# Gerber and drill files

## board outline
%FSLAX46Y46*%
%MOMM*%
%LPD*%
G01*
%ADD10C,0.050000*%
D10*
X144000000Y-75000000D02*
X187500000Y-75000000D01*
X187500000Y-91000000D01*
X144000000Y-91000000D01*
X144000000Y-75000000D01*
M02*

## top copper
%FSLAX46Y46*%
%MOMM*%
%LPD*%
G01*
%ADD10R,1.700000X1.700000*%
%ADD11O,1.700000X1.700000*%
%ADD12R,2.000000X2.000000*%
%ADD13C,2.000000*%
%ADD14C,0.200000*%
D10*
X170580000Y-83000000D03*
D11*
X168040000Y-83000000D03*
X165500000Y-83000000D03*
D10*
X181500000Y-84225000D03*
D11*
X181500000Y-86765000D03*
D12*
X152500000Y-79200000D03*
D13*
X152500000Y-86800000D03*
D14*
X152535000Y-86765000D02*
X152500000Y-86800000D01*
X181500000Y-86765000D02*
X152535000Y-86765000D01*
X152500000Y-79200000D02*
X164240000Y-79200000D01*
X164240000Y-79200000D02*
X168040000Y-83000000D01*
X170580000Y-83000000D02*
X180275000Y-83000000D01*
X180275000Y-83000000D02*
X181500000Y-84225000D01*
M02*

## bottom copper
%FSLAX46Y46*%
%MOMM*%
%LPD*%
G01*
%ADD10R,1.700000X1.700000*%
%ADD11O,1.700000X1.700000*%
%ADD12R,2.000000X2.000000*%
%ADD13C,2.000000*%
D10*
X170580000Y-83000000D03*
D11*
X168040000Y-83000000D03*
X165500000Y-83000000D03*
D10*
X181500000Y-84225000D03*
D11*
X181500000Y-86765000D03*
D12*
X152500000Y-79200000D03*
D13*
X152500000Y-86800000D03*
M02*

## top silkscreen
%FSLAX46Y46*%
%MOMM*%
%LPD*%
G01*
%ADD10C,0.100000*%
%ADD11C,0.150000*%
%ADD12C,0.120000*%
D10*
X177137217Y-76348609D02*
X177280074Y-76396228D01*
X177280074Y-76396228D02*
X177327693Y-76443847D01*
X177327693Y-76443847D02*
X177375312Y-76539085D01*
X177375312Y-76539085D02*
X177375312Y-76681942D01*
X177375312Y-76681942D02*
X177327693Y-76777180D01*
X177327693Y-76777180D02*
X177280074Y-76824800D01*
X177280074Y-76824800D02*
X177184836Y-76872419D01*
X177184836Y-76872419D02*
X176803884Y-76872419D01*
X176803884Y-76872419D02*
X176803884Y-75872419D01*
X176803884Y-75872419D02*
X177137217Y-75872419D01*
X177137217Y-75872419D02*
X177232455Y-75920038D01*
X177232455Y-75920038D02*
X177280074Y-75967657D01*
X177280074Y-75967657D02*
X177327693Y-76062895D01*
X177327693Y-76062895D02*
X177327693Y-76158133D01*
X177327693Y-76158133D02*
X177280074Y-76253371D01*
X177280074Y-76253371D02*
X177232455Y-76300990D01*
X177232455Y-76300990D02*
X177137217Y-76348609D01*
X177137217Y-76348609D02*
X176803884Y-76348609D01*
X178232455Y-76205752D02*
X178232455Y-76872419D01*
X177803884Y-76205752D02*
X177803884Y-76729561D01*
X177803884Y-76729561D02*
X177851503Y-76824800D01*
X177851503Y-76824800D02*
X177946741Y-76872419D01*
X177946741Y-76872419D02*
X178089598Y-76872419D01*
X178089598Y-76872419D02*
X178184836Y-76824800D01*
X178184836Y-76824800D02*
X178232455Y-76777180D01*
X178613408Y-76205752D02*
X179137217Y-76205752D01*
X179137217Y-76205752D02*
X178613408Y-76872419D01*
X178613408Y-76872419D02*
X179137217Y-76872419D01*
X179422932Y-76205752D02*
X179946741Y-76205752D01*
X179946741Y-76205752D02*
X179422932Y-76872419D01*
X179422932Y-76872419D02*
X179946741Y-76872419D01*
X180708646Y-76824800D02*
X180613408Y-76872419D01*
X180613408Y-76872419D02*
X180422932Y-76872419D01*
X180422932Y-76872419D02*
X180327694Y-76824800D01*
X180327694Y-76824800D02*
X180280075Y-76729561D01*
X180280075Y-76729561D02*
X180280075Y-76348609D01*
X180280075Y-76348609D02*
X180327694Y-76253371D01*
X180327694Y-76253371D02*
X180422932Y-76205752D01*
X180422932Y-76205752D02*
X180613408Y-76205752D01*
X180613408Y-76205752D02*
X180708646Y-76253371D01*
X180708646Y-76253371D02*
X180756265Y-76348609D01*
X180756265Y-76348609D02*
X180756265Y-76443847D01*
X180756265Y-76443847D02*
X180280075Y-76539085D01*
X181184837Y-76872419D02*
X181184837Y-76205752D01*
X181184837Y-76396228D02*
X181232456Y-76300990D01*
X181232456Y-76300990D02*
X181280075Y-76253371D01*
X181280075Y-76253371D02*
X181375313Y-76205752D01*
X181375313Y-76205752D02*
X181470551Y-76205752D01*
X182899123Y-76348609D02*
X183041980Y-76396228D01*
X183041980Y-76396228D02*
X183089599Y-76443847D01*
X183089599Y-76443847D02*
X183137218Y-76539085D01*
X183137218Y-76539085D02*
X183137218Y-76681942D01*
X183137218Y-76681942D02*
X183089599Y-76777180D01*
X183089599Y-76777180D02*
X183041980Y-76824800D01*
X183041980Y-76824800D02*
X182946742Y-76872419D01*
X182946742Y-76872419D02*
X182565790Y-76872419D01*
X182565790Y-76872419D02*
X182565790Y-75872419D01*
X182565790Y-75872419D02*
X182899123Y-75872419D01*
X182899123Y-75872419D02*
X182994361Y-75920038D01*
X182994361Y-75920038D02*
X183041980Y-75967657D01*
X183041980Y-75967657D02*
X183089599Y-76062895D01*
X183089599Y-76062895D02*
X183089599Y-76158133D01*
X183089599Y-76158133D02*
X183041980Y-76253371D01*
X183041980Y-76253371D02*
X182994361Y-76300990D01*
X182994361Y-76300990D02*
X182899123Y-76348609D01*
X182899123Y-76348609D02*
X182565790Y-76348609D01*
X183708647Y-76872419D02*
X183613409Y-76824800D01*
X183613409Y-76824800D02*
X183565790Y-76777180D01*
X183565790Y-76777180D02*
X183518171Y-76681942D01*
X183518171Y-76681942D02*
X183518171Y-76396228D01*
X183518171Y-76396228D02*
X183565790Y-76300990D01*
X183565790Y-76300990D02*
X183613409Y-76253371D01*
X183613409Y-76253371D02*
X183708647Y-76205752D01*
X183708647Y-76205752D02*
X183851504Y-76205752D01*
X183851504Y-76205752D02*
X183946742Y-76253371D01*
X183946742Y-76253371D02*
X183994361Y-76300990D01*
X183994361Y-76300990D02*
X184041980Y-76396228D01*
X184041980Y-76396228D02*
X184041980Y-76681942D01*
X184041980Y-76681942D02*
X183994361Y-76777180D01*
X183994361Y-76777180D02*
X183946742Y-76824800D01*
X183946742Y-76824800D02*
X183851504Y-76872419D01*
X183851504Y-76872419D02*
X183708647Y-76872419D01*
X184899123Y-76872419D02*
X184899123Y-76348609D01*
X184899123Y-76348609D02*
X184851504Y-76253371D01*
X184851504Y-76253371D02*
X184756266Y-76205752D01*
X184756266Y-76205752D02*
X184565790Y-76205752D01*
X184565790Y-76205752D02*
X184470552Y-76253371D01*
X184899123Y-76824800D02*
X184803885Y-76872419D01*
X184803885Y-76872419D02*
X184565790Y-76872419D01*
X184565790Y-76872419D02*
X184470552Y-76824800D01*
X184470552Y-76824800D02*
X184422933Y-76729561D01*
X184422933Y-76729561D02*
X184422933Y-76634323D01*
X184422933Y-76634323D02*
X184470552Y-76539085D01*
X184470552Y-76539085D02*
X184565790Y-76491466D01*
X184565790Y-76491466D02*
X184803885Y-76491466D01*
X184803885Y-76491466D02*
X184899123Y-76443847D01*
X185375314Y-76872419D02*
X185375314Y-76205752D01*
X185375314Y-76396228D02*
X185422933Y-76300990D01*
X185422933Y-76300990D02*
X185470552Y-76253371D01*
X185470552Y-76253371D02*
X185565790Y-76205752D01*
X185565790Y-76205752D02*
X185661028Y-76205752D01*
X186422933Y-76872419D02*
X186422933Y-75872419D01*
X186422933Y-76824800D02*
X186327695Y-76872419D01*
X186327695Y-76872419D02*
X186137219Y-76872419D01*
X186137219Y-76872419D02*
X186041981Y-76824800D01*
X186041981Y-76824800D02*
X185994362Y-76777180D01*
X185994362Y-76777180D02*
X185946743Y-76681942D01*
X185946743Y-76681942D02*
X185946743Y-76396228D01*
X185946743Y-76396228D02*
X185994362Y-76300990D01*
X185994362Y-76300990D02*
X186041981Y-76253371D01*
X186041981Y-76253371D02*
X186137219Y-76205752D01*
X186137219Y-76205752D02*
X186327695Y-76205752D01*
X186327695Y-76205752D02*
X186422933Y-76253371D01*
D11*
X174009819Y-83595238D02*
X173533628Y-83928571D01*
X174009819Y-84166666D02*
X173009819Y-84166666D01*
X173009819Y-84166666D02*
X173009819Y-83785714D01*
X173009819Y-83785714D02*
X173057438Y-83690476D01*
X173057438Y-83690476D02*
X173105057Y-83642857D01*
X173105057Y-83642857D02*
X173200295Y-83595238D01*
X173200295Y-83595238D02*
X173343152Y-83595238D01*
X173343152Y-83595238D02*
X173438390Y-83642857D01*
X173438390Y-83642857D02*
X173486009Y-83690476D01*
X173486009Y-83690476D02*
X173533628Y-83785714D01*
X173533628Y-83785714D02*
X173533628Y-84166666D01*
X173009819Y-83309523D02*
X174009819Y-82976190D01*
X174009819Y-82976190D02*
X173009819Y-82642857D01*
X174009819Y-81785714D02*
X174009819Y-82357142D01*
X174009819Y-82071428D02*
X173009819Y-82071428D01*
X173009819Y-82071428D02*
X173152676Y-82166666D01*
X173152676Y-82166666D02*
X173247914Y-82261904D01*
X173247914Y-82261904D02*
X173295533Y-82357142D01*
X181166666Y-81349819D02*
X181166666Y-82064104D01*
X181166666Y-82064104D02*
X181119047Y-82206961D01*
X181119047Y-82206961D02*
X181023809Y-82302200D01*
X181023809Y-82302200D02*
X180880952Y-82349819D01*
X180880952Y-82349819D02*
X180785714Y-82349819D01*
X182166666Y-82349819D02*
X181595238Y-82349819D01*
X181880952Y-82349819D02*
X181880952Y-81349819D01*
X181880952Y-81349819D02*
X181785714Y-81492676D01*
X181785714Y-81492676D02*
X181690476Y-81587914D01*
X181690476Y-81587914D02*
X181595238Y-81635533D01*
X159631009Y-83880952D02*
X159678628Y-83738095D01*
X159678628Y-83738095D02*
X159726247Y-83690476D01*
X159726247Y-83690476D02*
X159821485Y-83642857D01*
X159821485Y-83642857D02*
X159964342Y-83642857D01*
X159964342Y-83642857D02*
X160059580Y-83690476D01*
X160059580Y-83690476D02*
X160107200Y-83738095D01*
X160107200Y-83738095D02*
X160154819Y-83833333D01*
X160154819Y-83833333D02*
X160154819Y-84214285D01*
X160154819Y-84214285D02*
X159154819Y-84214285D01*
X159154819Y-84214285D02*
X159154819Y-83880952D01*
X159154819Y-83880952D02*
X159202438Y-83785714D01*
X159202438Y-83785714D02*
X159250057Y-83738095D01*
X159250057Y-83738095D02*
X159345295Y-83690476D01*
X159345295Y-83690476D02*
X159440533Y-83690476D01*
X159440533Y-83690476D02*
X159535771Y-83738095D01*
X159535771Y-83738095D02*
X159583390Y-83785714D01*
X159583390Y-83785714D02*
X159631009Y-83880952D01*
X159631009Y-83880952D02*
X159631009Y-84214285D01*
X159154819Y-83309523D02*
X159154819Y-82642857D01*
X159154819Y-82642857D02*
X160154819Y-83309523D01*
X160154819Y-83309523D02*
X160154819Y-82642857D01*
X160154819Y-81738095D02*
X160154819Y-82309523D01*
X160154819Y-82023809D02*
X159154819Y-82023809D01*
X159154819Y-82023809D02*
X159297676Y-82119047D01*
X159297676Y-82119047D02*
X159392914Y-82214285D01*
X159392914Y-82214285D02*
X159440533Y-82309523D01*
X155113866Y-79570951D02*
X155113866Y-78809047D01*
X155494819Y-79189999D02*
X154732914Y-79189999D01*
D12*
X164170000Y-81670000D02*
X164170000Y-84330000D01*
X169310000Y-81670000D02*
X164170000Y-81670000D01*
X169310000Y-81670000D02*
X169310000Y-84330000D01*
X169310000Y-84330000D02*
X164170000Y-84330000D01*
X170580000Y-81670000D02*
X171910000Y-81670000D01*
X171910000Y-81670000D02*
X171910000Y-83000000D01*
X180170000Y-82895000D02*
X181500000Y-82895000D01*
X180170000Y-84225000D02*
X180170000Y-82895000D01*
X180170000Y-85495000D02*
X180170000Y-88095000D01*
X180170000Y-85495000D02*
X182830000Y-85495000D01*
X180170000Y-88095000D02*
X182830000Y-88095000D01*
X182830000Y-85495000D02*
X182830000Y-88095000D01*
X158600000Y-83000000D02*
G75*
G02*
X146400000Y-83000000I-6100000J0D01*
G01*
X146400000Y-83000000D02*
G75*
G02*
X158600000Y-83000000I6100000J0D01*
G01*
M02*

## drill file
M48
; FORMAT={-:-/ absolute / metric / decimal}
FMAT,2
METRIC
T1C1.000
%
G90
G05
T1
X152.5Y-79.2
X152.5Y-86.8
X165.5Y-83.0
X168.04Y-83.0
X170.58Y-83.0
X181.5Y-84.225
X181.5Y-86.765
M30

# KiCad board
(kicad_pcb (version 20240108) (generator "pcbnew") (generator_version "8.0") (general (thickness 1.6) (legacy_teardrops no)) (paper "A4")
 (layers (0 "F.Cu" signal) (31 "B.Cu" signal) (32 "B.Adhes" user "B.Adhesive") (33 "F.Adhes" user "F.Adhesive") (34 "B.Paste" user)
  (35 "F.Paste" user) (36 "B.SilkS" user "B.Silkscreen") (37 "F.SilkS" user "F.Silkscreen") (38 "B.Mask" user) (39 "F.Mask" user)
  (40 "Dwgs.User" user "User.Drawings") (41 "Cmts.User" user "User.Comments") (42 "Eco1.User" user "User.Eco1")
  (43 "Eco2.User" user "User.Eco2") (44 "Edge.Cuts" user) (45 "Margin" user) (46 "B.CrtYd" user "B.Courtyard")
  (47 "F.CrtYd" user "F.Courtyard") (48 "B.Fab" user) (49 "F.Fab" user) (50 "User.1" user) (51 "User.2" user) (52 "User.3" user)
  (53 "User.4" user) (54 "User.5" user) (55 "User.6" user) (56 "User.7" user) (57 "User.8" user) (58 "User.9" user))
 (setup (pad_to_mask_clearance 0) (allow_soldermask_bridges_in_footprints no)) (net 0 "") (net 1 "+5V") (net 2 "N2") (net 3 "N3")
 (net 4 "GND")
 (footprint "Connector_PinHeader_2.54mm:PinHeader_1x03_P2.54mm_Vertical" (layer "F.Cu") (at 170.58 83 -90)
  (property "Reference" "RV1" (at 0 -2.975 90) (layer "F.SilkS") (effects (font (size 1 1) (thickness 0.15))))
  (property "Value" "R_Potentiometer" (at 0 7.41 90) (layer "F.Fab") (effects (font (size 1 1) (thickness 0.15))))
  (fp_line (start -1.33 6.41) (end 1.33 6.41) (stroke (width 0.12) (type solid)) (layer "F.SilkS"))
  (fp_line (start -1.33 1.27) (end -1.33 6.41) (stroke (width 0.12) (type solid)) (layer "F.SilkS"))
  (fp_line (start -1.33 1.27) (end 1.33 1.27) (stroke (width 0.12) (type solid)) (layer "F.SilkS"))
  (fp_line (start 1.33 1.27) (end 1.33 6.41) (stroke (width 0.12) (type solid)) (layer "F.SilkS"))
  (fp_line (start -1.33 0) (end -1.33 -1.33) (stroke (width 0.12) (type solid)) (layer "F.SilkS"))
  (fp_line (start -1.33 -1.33) (end 0 -1.33) (stroke (width 0.12) (type solid)) (layer "F.SilkS"))
  (pad "1" thru_hole rect (at 0 0 270) (size 1.7 1.7) (drill 1) (layers "*.Cu" "*.Mask") (remove_unused_layers no) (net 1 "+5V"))
  (pad "2" thru_hole oval (at 0 2.54 270) (size 1.7 1.7) (drill 1) (layers "*.Cu" "*.Mask") (remove_unused_layers no) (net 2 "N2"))
  (pad "3" thru_hole oval (at 0 5.08 270) (size 1.7 1.7) (drill 1) (layers "*.Cu" "*.Mask") (remove_unused_layers no) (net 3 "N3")))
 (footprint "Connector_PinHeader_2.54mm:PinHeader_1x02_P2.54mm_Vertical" (layer "F.Cu") (at 181.5 84.225)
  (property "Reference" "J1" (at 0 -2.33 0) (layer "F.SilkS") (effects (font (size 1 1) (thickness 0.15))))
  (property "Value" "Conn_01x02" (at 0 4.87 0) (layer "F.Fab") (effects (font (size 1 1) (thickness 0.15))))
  (fp_line (start -1.33 -1.33) (end 0 -1.33) (stroke (width 0.12) (type solid)) (layer "F.SilkS"))
  (fp_line (start -1.33 0) (end -1.33 -1.33) (stroke (width 0.12) (type solid)) (layer "F.SilkS"))
  (fp_line (start -1.33 1.27) (end -1.33 3.87) (stroke (width 0.12) (type solid)) (layer "F.SilkS"))
  (fp_line (start -1.33 1.27) (end 1.33 1.27) (stroke (width 0.12) (type solid)) (layer "F.SilkS"))
  (fp_line (start -1.33 3.87) (end 1.33 3.87) (stroke (width 0.12) (type solid)) (layer "F.SilkS"))
  (fp_line (start 1.33 1.27) (end 1.33 3.87) (stroke (width 0.12) (type solid)) (layer "F.SilkS"))
  (pad "1" thru_hole rect (at 0 0) (size 1.7 1.7) (drill 1) (layers "*.Cu" "*.Mask") (remove_unused_layers no) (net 1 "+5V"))
  (pad "2" thru_hole oval (at 0 2.54) (size 1.7 1.7) (drill 1) (layers "*.Cu" "*.Mask") (remove_unused_layers no) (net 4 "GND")))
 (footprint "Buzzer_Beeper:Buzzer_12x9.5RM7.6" (layer "F.Cu") (at 152.5 79.2 -90)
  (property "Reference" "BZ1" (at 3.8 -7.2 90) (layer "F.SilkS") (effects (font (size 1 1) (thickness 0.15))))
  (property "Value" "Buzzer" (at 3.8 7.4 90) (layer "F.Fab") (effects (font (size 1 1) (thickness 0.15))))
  (fp_circle (center 3.8 0) (end 9.9 0) (stroke (width 0.12) (type solid)) (fill none) (layer "F.SilkS"))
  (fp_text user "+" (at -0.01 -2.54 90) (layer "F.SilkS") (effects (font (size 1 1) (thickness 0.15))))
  (pad "1" thru_hole rect (at 0 0 270) (size 2 2) (drill 1) (layers "*.Cu" "*.Mask") (remove_unused_layers no) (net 2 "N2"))
  (pad "2" thru_hole circle (at 7.6 0 270) (size 2 2) (drill 1) (layers "*.Cu" "*.Mask") (remove_unused_layers no) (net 4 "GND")))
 (gr_poly (pts (xy 144 75) (xy 187.5 75) (xy 187.5 91) (xy 144 91)) (stroke (width 0.05) (type solid)) (fill none) (layer "Edge.Cuts"))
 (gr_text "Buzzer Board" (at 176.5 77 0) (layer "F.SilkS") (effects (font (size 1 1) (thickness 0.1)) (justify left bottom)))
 (segment (start 152.535 86.765) (end 152.5 86.8) (width 0.2) (layer "F.Cu") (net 4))
 (segment (start 181.5 86.765) (end 152.535 86.765) (width 0.2) (layer "F.Cu") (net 4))
 (segment (start 152.5 79.2) (end 164.24 79.2) (width 0.2) (layer "F.Cu") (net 2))
 (segment (start 164.24 79.2) (end 168.04 83) (width 0.2) (layer "F.Cu") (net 2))
 (segment (start 170.58 83) (end 180.275 83) (width 0.2) (layer "F.Cu") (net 1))
 (segment (start 180.275 83) (end 181.5 84.225) (width 0.2) (layer "F.Cu") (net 1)))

